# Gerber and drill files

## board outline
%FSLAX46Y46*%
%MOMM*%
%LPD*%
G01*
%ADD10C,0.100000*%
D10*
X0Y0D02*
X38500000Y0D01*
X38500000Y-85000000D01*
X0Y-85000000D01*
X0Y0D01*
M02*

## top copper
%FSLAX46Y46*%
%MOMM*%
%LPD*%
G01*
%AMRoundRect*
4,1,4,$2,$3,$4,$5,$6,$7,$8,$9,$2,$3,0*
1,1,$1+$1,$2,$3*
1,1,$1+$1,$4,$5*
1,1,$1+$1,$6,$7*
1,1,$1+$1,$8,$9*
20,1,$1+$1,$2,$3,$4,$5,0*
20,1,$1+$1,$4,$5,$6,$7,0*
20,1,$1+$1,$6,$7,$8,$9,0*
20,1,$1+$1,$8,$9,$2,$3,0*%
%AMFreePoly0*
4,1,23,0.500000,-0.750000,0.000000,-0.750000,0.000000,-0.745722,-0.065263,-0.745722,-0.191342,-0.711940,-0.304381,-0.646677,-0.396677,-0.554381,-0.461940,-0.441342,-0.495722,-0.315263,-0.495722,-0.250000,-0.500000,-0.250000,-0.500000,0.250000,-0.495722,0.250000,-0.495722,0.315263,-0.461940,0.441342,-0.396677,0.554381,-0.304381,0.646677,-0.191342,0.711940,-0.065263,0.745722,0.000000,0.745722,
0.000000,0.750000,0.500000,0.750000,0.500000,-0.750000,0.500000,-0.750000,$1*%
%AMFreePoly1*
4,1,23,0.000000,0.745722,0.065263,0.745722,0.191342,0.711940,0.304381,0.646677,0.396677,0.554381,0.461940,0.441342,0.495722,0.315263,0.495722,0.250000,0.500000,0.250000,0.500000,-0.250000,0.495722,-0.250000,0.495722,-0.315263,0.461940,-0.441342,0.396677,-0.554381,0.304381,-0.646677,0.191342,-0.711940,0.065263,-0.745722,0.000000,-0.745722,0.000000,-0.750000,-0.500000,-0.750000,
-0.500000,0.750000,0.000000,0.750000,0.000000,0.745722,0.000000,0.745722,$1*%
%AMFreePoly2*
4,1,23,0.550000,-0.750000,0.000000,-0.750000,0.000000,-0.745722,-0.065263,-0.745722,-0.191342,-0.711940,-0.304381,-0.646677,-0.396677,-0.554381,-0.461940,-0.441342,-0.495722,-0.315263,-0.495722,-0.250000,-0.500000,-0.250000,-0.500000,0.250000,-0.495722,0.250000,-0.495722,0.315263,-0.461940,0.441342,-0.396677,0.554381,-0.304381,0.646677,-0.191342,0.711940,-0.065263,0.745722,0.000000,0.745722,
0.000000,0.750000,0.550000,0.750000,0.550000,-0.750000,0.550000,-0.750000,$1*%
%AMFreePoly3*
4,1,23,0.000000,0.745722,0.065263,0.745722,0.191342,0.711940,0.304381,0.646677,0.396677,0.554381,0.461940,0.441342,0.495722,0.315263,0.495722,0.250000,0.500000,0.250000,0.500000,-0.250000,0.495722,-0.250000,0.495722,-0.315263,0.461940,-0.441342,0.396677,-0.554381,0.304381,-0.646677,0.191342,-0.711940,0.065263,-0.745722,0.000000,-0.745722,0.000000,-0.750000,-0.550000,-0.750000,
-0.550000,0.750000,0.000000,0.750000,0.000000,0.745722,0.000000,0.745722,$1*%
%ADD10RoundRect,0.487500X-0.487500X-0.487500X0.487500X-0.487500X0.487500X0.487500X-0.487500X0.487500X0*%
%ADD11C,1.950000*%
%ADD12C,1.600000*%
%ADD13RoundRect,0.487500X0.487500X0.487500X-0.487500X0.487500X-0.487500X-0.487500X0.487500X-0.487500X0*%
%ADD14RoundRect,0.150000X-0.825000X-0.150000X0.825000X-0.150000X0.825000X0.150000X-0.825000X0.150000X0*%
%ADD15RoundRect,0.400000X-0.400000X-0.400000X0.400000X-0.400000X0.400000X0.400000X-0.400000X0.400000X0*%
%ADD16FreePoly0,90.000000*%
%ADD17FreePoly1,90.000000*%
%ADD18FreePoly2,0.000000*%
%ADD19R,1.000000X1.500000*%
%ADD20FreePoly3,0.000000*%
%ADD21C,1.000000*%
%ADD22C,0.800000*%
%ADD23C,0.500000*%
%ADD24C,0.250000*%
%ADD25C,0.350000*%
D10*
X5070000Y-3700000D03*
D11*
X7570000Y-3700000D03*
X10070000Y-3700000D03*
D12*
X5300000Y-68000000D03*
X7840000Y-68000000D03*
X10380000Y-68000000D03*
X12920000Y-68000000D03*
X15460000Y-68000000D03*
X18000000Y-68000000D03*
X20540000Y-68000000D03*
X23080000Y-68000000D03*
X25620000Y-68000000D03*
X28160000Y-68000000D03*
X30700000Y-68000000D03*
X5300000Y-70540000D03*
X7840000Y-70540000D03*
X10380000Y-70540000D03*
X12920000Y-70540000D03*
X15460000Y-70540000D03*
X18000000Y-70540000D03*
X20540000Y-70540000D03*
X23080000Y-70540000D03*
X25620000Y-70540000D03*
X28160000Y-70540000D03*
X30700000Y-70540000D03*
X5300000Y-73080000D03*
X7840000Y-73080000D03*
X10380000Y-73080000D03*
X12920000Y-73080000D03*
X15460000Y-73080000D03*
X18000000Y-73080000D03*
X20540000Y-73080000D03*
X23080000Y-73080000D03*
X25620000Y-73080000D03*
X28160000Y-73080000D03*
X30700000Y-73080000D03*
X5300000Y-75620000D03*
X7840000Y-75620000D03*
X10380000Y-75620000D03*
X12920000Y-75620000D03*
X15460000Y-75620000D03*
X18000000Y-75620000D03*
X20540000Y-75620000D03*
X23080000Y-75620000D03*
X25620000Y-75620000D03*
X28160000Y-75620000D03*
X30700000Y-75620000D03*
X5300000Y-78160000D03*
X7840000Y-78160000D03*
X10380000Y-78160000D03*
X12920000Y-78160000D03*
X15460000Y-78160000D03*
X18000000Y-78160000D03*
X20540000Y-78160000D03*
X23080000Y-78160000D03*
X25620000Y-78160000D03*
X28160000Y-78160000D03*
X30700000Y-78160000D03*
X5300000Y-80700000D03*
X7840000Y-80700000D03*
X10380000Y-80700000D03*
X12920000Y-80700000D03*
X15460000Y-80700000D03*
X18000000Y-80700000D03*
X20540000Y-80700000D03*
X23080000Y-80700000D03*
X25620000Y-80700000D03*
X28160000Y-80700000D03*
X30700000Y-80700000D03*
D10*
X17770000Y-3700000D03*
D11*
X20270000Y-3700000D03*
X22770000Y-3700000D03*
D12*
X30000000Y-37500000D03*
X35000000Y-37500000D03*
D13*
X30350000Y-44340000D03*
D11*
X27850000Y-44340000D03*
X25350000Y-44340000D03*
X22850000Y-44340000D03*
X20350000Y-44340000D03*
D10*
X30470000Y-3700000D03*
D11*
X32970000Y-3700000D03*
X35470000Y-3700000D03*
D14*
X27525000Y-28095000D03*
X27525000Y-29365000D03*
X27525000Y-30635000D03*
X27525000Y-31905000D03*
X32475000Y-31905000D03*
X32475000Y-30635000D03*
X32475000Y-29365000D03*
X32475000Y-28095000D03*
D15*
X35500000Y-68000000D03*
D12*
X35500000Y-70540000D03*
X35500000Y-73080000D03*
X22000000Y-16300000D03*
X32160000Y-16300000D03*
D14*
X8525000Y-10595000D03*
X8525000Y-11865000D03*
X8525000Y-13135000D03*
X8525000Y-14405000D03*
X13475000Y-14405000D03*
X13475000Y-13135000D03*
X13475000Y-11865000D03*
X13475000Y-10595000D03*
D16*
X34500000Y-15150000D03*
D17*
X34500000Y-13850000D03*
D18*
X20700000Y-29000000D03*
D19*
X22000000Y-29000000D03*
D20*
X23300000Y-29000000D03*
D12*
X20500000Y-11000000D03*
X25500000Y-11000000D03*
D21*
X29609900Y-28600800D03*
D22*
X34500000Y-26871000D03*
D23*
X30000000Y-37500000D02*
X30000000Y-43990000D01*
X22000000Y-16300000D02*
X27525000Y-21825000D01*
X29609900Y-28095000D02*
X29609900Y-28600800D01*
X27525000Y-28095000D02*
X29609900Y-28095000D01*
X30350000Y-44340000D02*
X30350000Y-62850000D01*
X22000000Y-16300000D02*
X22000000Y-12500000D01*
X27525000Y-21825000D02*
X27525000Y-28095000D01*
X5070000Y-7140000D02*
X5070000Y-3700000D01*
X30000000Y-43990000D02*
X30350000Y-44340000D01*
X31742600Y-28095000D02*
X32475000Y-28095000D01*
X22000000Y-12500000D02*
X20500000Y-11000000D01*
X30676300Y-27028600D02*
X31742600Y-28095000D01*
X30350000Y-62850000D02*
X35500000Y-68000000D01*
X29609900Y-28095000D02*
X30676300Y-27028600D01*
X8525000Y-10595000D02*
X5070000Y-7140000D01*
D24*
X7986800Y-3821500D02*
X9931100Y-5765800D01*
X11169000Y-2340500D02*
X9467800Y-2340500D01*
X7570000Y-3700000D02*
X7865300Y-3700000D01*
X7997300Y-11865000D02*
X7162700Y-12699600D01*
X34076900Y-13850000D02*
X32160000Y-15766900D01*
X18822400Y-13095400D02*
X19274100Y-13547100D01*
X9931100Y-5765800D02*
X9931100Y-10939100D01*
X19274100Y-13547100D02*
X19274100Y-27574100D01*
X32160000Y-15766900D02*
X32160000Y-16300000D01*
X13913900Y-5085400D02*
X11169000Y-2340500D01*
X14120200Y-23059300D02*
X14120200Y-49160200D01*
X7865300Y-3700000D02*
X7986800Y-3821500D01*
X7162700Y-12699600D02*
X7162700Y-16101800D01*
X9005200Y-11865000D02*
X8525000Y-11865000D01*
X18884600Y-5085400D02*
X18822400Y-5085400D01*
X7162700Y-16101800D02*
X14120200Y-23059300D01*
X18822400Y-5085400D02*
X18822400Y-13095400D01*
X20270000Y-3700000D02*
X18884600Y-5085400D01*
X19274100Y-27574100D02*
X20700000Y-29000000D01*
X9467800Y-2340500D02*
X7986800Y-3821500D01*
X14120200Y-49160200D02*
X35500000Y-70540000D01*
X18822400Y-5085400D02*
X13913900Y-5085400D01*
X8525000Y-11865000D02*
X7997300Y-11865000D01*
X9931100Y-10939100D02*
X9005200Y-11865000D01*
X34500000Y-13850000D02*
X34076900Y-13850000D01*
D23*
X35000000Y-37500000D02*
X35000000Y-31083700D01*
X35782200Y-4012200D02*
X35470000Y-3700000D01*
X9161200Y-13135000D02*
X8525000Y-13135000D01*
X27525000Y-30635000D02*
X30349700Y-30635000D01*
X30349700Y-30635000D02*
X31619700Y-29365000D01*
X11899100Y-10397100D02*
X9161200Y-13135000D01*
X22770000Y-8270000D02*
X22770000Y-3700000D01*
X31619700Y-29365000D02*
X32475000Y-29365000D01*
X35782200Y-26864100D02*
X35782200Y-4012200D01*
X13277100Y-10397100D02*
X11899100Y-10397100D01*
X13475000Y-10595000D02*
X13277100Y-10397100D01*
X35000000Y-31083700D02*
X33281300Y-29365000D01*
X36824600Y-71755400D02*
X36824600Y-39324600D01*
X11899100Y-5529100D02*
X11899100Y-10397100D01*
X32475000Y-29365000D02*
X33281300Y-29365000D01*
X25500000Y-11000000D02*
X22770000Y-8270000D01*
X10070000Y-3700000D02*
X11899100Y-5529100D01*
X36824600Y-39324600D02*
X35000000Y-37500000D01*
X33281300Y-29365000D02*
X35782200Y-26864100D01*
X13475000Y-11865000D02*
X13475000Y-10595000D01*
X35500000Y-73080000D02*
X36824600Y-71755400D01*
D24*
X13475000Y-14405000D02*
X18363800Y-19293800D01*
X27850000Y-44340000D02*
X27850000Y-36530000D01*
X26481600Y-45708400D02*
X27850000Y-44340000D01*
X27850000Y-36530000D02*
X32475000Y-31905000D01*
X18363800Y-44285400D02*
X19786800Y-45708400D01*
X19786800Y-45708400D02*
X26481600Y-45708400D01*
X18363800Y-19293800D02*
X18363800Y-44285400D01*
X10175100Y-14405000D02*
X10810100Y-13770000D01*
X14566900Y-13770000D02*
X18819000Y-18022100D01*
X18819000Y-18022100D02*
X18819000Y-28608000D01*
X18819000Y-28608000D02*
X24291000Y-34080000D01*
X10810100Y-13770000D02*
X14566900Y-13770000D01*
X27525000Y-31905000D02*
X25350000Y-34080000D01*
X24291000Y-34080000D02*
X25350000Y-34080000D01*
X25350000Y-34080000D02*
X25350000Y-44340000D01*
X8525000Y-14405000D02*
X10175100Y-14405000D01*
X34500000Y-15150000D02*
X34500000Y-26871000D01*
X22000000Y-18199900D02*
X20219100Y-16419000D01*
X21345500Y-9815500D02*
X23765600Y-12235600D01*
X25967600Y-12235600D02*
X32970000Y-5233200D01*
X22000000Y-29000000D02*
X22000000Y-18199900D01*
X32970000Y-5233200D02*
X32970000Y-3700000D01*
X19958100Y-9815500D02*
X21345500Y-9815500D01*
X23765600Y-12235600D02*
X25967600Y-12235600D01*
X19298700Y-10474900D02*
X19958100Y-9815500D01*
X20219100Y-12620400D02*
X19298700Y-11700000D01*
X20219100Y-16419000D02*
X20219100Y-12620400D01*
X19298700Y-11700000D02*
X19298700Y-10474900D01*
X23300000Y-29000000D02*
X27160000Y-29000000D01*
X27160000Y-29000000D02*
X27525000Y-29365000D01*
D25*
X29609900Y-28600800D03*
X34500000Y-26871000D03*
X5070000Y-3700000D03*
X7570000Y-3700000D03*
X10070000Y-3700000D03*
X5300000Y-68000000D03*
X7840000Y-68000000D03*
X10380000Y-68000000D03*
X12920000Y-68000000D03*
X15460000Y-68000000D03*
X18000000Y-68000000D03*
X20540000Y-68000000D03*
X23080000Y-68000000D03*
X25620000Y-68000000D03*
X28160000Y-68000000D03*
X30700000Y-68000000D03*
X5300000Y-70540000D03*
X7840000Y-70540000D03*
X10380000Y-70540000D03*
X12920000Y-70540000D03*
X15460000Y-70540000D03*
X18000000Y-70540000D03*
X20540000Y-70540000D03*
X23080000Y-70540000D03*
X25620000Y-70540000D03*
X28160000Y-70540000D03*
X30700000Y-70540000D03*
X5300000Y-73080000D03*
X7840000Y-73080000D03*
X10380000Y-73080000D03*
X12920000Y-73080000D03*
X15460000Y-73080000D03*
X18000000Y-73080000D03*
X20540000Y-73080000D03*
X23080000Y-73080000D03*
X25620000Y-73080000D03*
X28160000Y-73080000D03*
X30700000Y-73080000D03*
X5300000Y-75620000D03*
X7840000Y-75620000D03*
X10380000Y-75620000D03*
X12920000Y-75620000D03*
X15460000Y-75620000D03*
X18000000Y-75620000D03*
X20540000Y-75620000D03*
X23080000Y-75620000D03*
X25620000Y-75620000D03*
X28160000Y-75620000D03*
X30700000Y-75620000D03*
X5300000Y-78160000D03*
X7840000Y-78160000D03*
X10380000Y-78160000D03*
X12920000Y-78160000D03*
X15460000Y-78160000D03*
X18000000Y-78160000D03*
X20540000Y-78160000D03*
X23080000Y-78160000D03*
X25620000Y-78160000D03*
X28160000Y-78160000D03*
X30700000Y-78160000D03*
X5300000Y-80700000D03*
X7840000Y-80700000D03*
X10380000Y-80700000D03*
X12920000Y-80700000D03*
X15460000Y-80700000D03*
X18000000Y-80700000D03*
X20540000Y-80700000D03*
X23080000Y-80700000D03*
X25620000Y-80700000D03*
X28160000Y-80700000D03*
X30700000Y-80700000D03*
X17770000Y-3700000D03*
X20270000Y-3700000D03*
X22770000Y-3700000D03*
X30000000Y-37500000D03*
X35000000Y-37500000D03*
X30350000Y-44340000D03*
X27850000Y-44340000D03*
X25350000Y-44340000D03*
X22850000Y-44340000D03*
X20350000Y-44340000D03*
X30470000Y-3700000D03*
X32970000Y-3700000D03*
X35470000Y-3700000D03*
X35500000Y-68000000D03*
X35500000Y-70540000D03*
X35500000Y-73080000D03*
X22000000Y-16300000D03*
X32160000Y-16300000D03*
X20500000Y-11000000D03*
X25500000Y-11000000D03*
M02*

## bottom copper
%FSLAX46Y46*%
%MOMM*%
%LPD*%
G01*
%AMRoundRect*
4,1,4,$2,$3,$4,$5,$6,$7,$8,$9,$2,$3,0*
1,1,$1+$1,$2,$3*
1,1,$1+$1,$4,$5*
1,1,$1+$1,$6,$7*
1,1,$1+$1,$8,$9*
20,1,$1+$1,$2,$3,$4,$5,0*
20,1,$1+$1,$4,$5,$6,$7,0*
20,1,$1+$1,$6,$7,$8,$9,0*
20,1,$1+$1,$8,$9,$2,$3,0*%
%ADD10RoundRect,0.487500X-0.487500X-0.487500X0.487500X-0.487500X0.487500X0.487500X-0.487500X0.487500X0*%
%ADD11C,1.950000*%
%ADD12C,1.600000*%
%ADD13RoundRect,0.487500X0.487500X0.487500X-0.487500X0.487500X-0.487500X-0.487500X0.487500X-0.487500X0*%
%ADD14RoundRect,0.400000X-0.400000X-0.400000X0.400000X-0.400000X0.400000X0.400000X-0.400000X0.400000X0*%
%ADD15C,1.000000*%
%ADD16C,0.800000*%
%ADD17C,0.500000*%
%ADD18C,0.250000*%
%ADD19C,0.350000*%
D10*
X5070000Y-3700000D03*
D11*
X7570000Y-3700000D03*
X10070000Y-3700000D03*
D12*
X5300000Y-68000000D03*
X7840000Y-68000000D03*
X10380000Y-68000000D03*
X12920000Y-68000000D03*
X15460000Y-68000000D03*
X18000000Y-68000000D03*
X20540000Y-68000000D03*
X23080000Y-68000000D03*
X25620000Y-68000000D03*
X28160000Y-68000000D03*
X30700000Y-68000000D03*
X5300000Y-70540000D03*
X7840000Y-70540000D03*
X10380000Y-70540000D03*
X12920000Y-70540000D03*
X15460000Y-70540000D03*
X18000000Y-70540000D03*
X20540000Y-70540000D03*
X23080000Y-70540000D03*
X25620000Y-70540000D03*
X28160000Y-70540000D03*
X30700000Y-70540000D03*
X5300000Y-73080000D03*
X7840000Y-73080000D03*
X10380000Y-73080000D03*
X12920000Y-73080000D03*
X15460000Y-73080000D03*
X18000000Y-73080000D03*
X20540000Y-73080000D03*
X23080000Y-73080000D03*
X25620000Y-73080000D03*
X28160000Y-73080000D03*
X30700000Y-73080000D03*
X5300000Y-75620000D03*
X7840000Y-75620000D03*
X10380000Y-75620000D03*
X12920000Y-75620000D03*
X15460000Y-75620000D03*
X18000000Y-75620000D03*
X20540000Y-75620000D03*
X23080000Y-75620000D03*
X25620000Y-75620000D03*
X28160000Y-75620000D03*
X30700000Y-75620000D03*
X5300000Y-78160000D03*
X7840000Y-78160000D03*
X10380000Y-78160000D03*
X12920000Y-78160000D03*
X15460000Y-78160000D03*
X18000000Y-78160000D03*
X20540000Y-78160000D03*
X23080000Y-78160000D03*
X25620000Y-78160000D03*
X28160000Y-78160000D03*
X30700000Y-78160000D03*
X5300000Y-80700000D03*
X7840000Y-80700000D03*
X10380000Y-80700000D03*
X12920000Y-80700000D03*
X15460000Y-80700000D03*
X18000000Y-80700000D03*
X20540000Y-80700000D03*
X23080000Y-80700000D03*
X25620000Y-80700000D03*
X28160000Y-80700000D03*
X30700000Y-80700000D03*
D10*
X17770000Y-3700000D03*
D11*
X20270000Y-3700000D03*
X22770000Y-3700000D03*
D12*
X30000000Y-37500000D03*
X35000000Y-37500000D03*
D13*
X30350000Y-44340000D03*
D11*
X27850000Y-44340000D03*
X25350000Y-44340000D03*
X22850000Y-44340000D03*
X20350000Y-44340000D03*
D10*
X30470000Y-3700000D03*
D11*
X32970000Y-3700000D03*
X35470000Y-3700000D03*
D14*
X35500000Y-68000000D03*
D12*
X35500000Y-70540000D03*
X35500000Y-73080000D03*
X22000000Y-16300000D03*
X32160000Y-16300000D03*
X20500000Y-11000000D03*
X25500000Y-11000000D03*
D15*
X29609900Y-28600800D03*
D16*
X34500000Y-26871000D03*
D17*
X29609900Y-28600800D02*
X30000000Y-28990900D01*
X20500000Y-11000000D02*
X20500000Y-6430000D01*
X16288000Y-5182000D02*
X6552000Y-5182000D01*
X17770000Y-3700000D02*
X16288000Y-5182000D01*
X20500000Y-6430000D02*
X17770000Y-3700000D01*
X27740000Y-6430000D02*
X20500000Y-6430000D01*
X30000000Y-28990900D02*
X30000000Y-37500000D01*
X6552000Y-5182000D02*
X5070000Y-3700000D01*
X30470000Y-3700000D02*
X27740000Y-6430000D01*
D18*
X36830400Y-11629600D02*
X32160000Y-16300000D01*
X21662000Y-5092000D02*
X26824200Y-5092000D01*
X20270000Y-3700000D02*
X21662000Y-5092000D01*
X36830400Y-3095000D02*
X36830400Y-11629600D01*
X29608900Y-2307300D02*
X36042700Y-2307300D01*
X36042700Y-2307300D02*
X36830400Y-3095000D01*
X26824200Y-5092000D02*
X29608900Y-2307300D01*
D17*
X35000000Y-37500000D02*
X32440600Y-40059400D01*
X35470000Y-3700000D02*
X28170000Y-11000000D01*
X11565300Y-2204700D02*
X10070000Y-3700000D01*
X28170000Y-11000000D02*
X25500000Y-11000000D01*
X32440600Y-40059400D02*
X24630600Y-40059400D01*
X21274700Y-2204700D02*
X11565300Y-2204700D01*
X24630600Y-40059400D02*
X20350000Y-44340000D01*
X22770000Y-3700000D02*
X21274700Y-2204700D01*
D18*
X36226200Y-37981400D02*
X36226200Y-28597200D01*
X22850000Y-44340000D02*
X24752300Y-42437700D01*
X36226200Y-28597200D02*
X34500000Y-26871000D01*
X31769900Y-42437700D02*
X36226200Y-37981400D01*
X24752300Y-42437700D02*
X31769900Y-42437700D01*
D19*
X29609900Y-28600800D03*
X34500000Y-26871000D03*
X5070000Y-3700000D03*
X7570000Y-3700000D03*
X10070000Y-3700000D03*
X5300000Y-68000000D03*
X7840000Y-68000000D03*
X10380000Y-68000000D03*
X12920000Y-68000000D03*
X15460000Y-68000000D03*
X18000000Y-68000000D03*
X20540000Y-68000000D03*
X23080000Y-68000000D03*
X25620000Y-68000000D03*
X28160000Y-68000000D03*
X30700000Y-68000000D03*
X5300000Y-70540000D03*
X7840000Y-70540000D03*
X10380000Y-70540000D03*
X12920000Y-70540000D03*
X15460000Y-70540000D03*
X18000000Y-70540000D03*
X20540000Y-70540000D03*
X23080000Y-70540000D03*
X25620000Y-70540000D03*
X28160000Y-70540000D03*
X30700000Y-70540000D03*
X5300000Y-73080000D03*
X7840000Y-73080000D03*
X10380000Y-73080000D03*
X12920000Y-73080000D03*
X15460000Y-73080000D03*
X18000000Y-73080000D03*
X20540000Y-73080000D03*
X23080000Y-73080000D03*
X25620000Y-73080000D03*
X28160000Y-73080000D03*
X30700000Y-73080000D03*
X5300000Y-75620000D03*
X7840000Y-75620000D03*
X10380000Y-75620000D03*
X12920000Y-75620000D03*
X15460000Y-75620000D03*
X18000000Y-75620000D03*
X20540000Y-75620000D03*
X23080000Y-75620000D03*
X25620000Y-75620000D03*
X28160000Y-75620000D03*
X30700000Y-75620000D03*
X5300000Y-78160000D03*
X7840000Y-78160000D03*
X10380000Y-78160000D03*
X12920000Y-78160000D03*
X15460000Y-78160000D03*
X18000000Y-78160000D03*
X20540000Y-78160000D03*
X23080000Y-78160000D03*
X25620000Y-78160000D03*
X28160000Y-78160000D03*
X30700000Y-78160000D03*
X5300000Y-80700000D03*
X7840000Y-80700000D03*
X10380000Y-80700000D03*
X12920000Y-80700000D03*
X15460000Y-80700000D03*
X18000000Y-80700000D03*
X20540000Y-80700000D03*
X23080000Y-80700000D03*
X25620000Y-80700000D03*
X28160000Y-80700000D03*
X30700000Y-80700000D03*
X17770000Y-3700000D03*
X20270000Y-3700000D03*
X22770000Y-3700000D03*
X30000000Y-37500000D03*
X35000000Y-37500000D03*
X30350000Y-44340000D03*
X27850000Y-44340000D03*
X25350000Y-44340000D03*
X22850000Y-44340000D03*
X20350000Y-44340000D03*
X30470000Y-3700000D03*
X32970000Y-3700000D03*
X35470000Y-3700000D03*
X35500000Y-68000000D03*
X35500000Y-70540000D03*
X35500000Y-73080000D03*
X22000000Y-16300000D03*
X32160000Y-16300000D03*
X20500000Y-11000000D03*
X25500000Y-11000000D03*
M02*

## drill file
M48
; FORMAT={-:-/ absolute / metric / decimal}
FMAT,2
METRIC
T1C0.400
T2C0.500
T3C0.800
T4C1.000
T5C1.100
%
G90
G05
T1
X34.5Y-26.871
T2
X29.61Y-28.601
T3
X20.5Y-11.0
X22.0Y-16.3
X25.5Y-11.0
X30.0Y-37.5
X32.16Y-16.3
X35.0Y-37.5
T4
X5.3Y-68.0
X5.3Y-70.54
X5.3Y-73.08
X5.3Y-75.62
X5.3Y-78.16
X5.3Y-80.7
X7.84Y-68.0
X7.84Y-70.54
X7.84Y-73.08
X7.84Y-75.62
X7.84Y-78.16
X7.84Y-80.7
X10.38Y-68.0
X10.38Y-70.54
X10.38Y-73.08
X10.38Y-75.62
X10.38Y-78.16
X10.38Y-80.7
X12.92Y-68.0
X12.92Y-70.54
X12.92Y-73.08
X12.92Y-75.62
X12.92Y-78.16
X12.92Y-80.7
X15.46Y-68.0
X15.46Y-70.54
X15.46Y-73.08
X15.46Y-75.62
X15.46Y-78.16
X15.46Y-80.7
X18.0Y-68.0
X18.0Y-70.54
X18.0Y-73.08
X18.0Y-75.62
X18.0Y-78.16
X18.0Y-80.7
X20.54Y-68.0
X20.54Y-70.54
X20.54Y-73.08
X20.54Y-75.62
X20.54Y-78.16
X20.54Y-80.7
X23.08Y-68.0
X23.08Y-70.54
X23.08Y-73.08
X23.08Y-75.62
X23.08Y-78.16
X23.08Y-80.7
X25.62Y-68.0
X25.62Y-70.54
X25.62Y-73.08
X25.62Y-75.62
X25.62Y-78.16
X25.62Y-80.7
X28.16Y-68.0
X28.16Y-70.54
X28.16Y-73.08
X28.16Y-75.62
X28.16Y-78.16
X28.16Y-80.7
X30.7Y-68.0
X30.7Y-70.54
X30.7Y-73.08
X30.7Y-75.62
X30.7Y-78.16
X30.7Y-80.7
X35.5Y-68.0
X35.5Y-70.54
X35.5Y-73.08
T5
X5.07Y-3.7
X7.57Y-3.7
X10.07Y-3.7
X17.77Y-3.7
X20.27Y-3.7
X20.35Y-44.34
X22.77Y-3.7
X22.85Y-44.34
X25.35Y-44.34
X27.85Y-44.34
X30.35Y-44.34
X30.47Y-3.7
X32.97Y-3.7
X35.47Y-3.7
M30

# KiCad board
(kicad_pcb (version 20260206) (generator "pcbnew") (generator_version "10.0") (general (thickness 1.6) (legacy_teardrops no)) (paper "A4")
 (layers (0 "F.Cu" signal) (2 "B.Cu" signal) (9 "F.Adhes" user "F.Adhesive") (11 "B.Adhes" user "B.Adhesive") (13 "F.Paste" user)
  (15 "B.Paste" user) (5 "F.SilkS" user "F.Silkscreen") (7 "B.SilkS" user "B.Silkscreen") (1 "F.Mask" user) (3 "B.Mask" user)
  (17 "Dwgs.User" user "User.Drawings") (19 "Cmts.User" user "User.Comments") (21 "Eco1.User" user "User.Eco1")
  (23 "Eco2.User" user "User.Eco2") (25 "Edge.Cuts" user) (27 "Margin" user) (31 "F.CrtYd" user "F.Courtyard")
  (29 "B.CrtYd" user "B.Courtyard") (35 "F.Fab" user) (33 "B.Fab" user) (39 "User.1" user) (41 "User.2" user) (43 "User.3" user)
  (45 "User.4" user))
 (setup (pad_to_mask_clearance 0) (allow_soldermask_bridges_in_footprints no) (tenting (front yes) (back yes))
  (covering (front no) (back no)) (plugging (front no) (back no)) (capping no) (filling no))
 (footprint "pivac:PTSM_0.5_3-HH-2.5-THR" (layer "F.Cu") (at 7.57 3.7)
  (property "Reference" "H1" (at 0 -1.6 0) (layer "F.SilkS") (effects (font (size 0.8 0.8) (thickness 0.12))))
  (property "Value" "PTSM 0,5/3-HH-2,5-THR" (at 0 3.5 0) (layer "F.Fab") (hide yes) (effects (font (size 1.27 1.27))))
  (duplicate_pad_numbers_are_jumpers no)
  (pad "1" thru_hole roundrect (at -2.5 0) (size 1.95 1.95) (drill 1.1) (layers "*.Cu" "*.Mask") (remove_unused_layers no)
   (roundrect_rratio 0.25) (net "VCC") (thermal_bridge_angle 45))
  (pad "2" thru_hole circle (at 0 0) (size 1.95 1.95) (drill 1.1) (layers "*.Cu" "*.Mask") (remove_unused_layers no) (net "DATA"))
  (pad "3" thru_hole circle (at 2.5 0) (size 1.95 1.95) (drill 1.1) (layers "*.Cu" "*.Mask") (remove_unused_layers no) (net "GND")))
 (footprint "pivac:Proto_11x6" (layer "F.Cu") (at 5.3 68)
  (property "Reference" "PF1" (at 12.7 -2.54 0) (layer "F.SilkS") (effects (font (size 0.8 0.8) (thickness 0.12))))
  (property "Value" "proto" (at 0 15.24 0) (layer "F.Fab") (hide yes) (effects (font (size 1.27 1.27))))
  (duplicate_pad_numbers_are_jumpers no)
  (pad "1" thru_hole circle (at 0 0) (size 1.6 1.6) (drill 1) (layers "*.Cu" "*.Mask") (remove_unused_layers no))
  (pad "2" thru_hole circle (at 2.54 0) (size 1.6 1.6) (drill 1) (layers "*.Cu" "*.Mask") (remove_unused_layers no))
  (pad "3" thru_hole circle (at 5.08 0) (size 1.6 1.6) (drill 1) (layers "*.Cu" "*.Mask") (remove_unused_layers no))
  (pad "4" thru_hole circle (at 7.62 0) (size 1.6 1.6) (drill 1) (layers "*.Cu" "*.Mask") (remove_unused_layers no))
  (pad "5" thru_hole circle (at 10.16 0) (size 1.6 1.6) (drill 1) (layers "*.Cu" "*.Mask") (remove_unused_layers no))
  (pad "6" thru_hole circle (at 12.7 0) (size 1.6 1.6) (drill 1) (layers "*.Cu" "*.Mask") (remove_unused_layers no))
  (pad "7" thru_hole circle (at 15.24 0) (size 1.6 1.6) (drill 1) (layers "*.Cu" "*.Mask") (remove_unused_layers no))
  (pad "8" thru_hole circle (at 17.78 0) (size 1.6 1.6) (drill 1) (layers "*.Cu" "*.Mask") (remove_unused_layers no))
  (pad "9" thru_hole circle (at 20.32 0) (size 1.6 1.6) (drill 1) (layers "*.Cu" "*.Mask") (remove_unused_layers no))
  (pad "10" thru_hole circle (at 22.86 0) (size 1.6 1.6) (drill 1) (layers "*.Cu" "*.Mask") (remove_unused_layers no))
  (pad "11" thru_hole circle (at 25.4 0) (size 1.6 1.6) (drill 1) (layers "*.Cu" "*.Mask") (remove_unused_layers no))
  (pad "12" thru_hole circle (at 0 2.54) (size 1.6 1.6) (drill 1) (layers "*.Cu" "*.Mask") (remove_unused_layers no))
  (pad "13" thru_hole circle (at 2.54 2.54) (size 1.6 1.6) (drill 1) (layers "*.Cu" "*.Mask") (remove_unused_layers no))
  (pad "14" thru_hole circle (at 5.08 2.54) (size 1.6 1.6) (drill 1) (layers "*.Cu" "*.Mask") (remove_unused_layers no))
  (pad "15" thru_hole circle (at 7.62 2.54) (size 1.6 1.6) (drill 1) (layers "*.Cu" "*.Mask") (remove_unused_layers no))
  (pad "16" thru_hole circle (at 10.16 2.54) (size 1.6 1.6) (drill 1) (layers "*.Cu" "*.Mask") (remove_unused_layers no))
  (pad "17" thru_hole circle (at 12.7 2.54) (size 1.6 1.6) (drill 1) (layers "*.Cu" "*.Mask") (remove_unused_layers no))
  (pad "18" thru_hole circle (at 15.24 2.54) (size 1.6 1.6) (drill 1) (layers "*.Cu" "*.Mask") (remove_unused_layers no))
  (pad "19" thru_hole circle (at 17.78 2.54) (size 1.6 1.6) (drill 1) (layers "*.Cu" "*.Mask") (remove_unused_layers no))
  (pad "20" thru_hole circle (at 20.32 2.54) (size 1.6 1.6) (drill 1) (layers "*.Cu" "*.Mask") (remove_unused_layers no))
  (pad "21" thru_hole circle (at 22.86 2.54) (size 1.6 1.6) (drill 1) (layers "*.Cu" "*.Mask") (remove_unused_layers no))
  (pad "22" thru_hole circle (at 25.4 2.54) (size 1.6 1.6) (drill 1) (layers "*.Cu" "*.Mask") (remove_unused_layers no))
  (pad "23" thru_hole circle (at 0 5.08) (size 1.6 1.6) (drill 1) (layers "*.Cu" "*.Mask") (remove_unused_layers no))
  (pad "24" thru_hole circle (at 2.54 5.08) (size 1.6 1.6) (drill 1) (layers "*.Cu" "*.Mask") (remove_unused_layers no))
  (pad "25" thru_hole circle (at 5.08 5.08) (size 1.6 1.6) (drill 1) (layers "*.Cu" "*.Mask") (remove_unused_layers no))
  (pad "26" thru_hole circle (at 7.62 5.08) (size 1.6 1.6) (drill 1) (layers "*.Cu" "*.Mask") (remove_unused_layers no))
  (pad "27" thru_hole circle (at 10.16 5.08) (size 1.6 1.6) (drill 1) (layers "*.Cu" "*.Mask") (remove_unused_layers no))
  (pad "28" thru_hole circle (at 12.7 5.08) (size 1.6 1.6) (drill 1) (layers "*.Cu" "*.Mask") (remove_unused_layers no))
  (pad "29" thru_hole circle (at 15.24 5.08) (size 1.6 1.6) (drill 1) (layers "*.Cu" "*.Mask") (remove_unused_layers no))
  (pad "30" thru_hole circle (at 17.78 5.08) (size 1.6 1.6) (drill 1) (layers "*.Cu" "*.Mask") (remove_unused_layers no))
  (pad "31" thru_hole circle (at 20.32 5.08) (size 1.6 1.6) (drill 1) (layers "*.Cu" "*.Mask") (remove_unused_layers no))
  (pad "32" thru_hole circle (at 22.86 5.08) (size 1.6 1.6) (drill 1) (layers "*.Cu" "*.Mask") (remove_unused_layers no))
  (pad "33" thru_hole circle (at 25.4 5.08) (size 1.6 1.6) (drill 1) (layers "*.Cu" "*.Mask") (remove_unused_layers no))
  (pad "34" thru_hole circle (at 0 7.62) (size 1.6 1.6) (drill 1) (layers "*.Cu" "*.Mask") (remove_unused_layers no))
  (pad "35" thru_hole circle (at 2.54 7.62) (size 1.6 1.6) (drill 1) (layers "*.Cu" "*.Mask") (remove_unused_layers no))
  (pad "36" thru_hole circle (at 5.08 7.62) (size 1.6 1.6) (drill 1) (layers "*.Cu" "*.Mask") (remove_unused_layers no))
  (pad "37" thru_hole circle (at 7.62 7.62) (size 1.6 1.6) (drill 1) (layers "*.Cu" "*.Mask") (remove_unused_layers no))
  (pad "38" thru_hole circle (at 10.16 7.62) (size 1.6 1.6) (drill 1) (layers "*.Cu" "*.Mask") (remove_unused_layers no))
  (pad "39" thru_hole circle (at 12.7 7.62) (size 1.6 1.6) (drill 1) (layers "*.Cu" "*.Mask") (remove_unused_layers no))
  (pad "40" thru_hole circle (at 15.24 7.62) (size 1.6 1.6) (drill 1) (layers "*.Cu" "*.Mask") (remove_unused_layers no))
  (pad "41" thru_hole circle (at 17.78 7.62) (size 1.6 1.6) (drill 1) (layers "*.Cu" "*.Mask") (remove_unused_layers no))
  (pad "42" thru_hole circle (at 20.32 7.62) (size 1.6 1.6) (drill 1) (layers "*.Cu" "*.Mask") (remove_unused_layers no))
  (pad "43" thru_hole circle (at 22.86 7.62) (size 1.6 1.6) (drill 1) (layers "*.Cu" "*.Mask") (remove_unused_layers no))
  (pad "44" thru_hole circle (at 25.4 7.62) (size 1.6 1.6) (drill 1) (layers "*.Cu" "*.Mask") (remove_unused_layers no))
  (pad "45" thru_hole circle (at 0 10.16) (size 1.6 1.6) (drill 1) (layers "*.Cu" "*.Mask") (remove_unused_layers no))
  (pad "46" thru_hole circle (at 2.54 10.16) (size 1.6 1.6) (drill 1) (layers "*.Cu" "*.Mask") (remove_unused_layers no))
  (pad "47" thru_hole circle (at 5.08 10.16) (size 1.6 1.6) (drill 1) (layers "*.Cu" "*.Mask") (remove_unused_layers no))
  (pad "48" thru_hole circle (at 7.62 10.16) (size 1.6 1.6) (drill 1) (layers "*.Cu" "*.Mask") (remove_unused_layers no))
  (pad "49" thru_hole circle (at 10.16 10.16) (size 1.6 1.6) (drill 1) (layers "*.Cu" "*.Mask") (remove_unused_layers no))
  (pad "50" thru_hole circle (at 12.7 10.16) (size 1.6 1.6) (drill 1) (layers "*.Cu" "*.Mask") (remove_unused_layers no))
  (pad "51" thru_hole circle (at 15.24 10.16) (size 1.6 1.6) (drill 1) (layers "*.Cu" "*.Mask") (remove_unused_layers no))
  (pad "52" thru_hole circle (at 17.78 10.16) (size 1.6 1.6) (drill 1) (layers "*.Cu" "*.Mask") (remove_unused_layers no))
  (pad "53" thru_hole circle (at 20.32 10.16) (size 1.6 1.6) (drill 1) (layers "*.Cu" "*.Mask") (remove_unused_layers no))
  (pad "54" thru_hole circle (at 22.86 10.16) (size 1.6 1.6) (drill 1) (layers "*.Cu" "*.Mask") (remove_unused_layers no))
  (pad "55" thru_hole circle (at 25.4 10.16) (size 1.6 1.6) (drill 1) (layers "*.Cu" "*.Mask") (remove_unused_layers no))
  (pad "56" thru_hole circle (at 0 12.7) (size 1.6 1.6) (drill 1) (layers "*.Cu" "*.Mask") (remove_unused_layers no))
  (pad "57" thru_hole circle (at 2.54 12.7) (size 1.6 1.6) (drill 1) (layers "*.Cu" "*.Mask") (remove_unused_layers no))
  (pad "58" thru_hole circle (at 5.08 12.7) (size 1.6 1.6) (drill 1) (layers "*.Cu" "*.Mask") (remove_unused_layers no))
  (pad "59" thru_hole circle (at 7.62 12.7) (size 1.6 1.6) (drill 1) (layers "*.Cu" "*.Mask") (remove_unused_layers no))
  (pad "60" thru_hole circle (at 10.16 12.7) (size 1.6 1.6) (drill 1) (layers "*.Cu" "*.Mask") (remove_unused_layers no))
  (pad "61" thru_hole circle (at 12.7 12.7) (size 1.6 1.6) (drill 1) (layers "*.Cu" "*.Mask") (remove_unused_layers no))
  (pad "62" thru_hole circle (at 15.24 12.7) (size 1.6 1.6) (drill 1) (layers "*.Cu" "*.Mask") (remove_unused_layers no))
  (pad "63" thru_hole circle (at 17.78 12.7) (size 1.6 1.6) (drill 1) (layers "*.Cu" "*.Mask") (remove_unused_layers no))
  (pad "64" thru_hole circle (at 20.32 12.7) (size 1.6 1.6) (drill 1) (layers "*.Cu" "*.Mask") (remove_unused_layers no))
  (pad "65" thru_hole circle (at 22.86 12.7) (size 1.6 1.6) (drill 1) (layers "*.Cu" "*.Mask") (remove_unused_layers no))
  (pad "66" thru_hole circle (at 25.4 12.7) (size 1.6 1.6) (drill 1) (layers "*.Cu" "*.Mask") (remove_unused_layers no)))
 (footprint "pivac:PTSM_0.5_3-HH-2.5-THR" (layer "F.Cu") (at 20.27 3.7)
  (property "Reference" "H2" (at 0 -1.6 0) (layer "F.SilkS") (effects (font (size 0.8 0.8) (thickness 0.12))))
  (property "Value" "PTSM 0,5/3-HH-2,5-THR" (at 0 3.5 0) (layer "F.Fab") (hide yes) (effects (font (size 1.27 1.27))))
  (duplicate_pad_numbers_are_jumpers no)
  (pad "1" thru_hole roundrect (at -2.5 0) (size 1.95 1.95) (drill 1.1) (layers "*.Cu" "*.Mask") (remove_unused_layers no)
   (roundrect_rratio 0.25) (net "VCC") (thermal_bridge_angle 45))
  (pad "2" thru_hole circle (at 0 0) (size 1.95 1.95) (drill 1.1) (layers "*.Cu" "*.Mask") (remove_unused_layers no) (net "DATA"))
  (pad "3" thru_hole circle (at 2.5 0) (size 1.95 1.95) (drill 1.1) (layers "*.Cu" "*.Mask") (remove_unused_layers no) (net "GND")))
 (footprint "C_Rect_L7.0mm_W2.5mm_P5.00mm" (layer "F.Cu") (at 30 37.5)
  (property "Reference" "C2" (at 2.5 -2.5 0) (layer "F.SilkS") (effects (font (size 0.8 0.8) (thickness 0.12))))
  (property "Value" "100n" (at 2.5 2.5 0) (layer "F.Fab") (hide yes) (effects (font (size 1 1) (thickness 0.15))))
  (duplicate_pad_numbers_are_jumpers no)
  (pad "1" thru_hole circle (at 0 0) (size 1.6 1.6) (drill 0.8) (layers "*.Cu" "*.Mask") (remove_unused_layers no) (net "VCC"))
  (pad "2" thru_hole circle (at 5 0) (size 1.6 1.6) (drill 0.8) (layers "*.Cu" "*.Mask") (remove_unused_layers no) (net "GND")))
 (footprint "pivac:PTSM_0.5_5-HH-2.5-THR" (layer "F.Cu") (at 25.35 44.34 180)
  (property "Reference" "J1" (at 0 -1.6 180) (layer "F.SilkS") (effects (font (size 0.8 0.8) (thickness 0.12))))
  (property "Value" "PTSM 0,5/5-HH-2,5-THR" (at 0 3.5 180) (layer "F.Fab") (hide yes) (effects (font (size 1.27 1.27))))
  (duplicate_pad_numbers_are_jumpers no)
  (pad "1" thru_hole roundrect (at -5 0 180) (size 1.95 1.95) (drill 1.1) (layers "*.Cu" "*.Mask") (remove_unused_layers no)
   (roundrect_rratio 0.25) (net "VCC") (thermal_bridge_angle 45))
  (pad "2" thru_hole circle (at -2.5 0 180) (size 1.95 1.95) (drill 1.1) (layers "*.Cu" "*.Mask") (remove_unused_layers no) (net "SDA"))
  (pad "3" thru_hole circle (at 0 0 180) (size 1.95 1.95) (drill 1.1) (layers "*.Cu" "*.Mask") (remove_unused_layers no) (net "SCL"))
  (pad "4" thru_hole circle (at 2.5 0 180) (size 1.95 1.95) (drill 1.1) (layers "*.Cu" "*.Mask") (remove_unused_layers no) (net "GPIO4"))
  (pad "5" thru_hole circle (at 5 0 180) (size 1.95 1.95) (drill 1.1) (layers "*.Cu" "*.Mask") (remove_unused_layers no) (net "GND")))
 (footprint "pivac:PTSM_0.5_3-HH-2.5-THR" (layer "F.Cu") (at 32.97 3.7)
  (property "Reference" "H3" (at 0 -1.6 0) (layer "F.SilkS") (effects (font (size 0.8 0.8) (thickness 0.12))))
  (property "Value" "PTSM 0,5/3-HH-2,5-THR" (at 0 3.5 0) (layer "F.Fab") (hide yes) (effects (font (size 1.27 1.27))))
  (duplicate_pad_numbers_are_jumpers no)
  (pad "1" thru_hole roundrect (at -2.5 0) (size 1.95 1.95) (drill 1.1) (layers "*.Cu" "*.Mask") (remove_unused_layers no)
   (roundrect_rratio 0.25) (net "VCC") (thermal_bridge_angle 45))
  (pad "2" thru_hole circle (at 0 0) (size 1.95 1.95) (drill 1.1) (layers "*.Cu" "*.Mask") (remove_unused_layers no) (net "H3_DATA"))
  (pad "3" thru_hole circle (at 2.5 0) (size 1.95 1.95) (drill 1.1) (layers "*.Cu" "*.Mask") (remove_unused_layers no) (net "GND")))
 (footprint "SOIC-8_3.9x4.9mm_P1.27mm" (layer "F.Cu") (at 30 30)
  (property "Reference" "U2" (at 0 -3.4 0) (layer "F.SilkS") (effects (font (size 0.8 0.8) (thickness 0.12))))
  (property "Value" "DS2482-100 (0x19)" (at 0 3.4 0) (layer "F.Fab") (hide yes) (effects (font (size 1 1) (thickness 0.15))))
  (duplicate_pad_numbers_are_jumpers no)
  (pad "1" smd roundrect (at -2.475 -1.905) (size 1.95 0.6) (layers "F.Cu" "F.Mask" "F.Paste") (roundrect_rratio 0.25) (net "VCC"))
  (pad "2" smd roundrect (at -2.475 -0.635) (size 1.95 0.6) (layers "F.Cu" "F.Mask" "F.Paste") (roundrect_rratio 0.25) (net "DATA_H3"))
  (pad "3" smd roundrect (at -2.475 0.635) (size 1.95 0.6) (layers "F.Cu" "F.Mask" "F.Paste") (roundrect_rratio 0.25) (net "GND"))
  (pad "4" smd roundrect (at -2.475 1.905) (size 1.95 0.6) (layers "F.Cu" "F.Mask" "F.Paste") (roundrect_rratio 0.25) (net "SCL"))
  (pad "5" smd roundrect (at 2.475 1.905) (size 1.95 0.6) (layers "F.Cu" "F.Mask" "F.Paste") (roundrect_rratio 0.25) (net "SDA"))
  (pad "6" smd roundrect (at 2.475 0.635) (size 1.95 0.6) (layers "F.Cu" "F.Mask" "F.Paste") (roundrect_rratio 0.25))
  (pad "7" smd roundrect (at 2.475 -0.635) (size 1.95 0.6) (layers "F.Cu" "F.Mask" "F.Paste") (roundrect_rratio 0.25) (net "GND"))
  (pad "8" smd roundrect (at 2.475 -1.905) (size 1.95 0.6) (layers "F.Cu" "F.Mask" "F.Paste") (roundrect_rratio 0.25) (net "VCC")))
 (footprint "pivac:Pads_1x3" (layer "F.Cu") (at 35.5 68)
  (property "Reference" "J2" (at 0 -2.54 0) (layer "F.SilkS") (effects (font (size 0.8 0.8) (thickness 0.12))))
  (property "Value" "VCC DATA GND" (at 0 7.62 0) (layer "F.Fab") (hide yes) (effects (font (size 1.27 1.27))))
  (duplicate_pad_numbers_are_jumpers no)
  (pad "1" thru_hole roundrect (at 0 0) (size 1.6 1.6) (drill 1) (layers "*.Cu" "*.Mask") (remove_unused_layers no) (roundrect_rratio 0.25)
   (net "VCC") (thermal_bridge_angle 45))
  (pad "2" thru_hole circle (at 0 2.54) (size 1.6 1.6) (drill 1) (layers "*.Cu" "*.Mask") (remove_unused_layers no) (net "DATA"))
  (pad "3" thru_hole circle (at 0 5.08) (size 1.6 1.6) (drill 1) (layers "*.Cu" "*.Mask") (remove_unused_layers no) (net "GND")))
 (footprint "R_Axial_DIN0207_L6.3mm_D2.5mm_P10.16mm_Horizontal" (layer "F.Cu") (at 22 16.3)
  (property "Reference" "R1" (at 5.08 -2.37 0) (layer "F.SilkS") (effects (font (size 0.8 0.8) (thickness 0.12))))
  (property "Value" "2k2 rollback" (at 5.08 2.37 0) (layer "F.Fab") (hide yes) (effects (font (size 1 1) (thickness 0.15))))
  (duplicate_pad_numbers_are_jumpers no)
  (pad "1" thru_hole circle (at 0 0) (size 1.6 1.6) (drill 0.8) (layers "*.Cu" "*.Mask") (remove_unused_layers no) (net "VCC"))
  (pad "2" thru_hole circle (at 10.16 0) (size 1.6 1.6) (drill 0.8) (layers "*.Cu" "*.Mask") (remove_unused_layers no) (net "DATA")))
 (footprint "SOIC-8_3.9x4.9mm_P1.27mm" (layer "F.Cu") (at 11 12.5)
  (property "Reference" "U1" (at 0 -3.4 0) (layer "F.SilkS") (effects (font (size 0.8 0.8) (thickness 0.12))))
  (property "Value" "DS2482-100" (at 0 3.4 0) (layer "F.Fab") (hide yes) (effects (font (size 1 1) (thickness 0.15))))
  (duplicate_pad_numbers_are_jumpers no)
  (pad "1" smd roundrect (at -2.475 -1.905) (size 1.95 0.6) (layers "F.Cu" "F.Mask" "F.Paste") (roundrect_rratio 0.25) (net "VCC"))
  (pad "2" smd roundrect (at -2.475 -0.635) (size 1.95 0.6) (layers "F.Cu" "F.Mask" "F.Paste") (roundrect_rratio 0.25) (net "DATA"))
  (pad "3" smd roundrect (at -2.475 0.635) (size 1.95 0.6) (layers "F.Cu" "F.Mask" "F.Paste") (roundrect_rratio 0.25) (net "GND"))
  (pad "4" smd roundrect (at -2.475 1.905) (size 1.95 0.6) (layers "F.Cu" "F.Mask" "F.Paste") (roundrect_rratio 0.25) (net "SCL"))
  (pad "5" smd roundrect (at 2.475 1.905) (size 1.95 0.6) (layers "F.Cu" "F.Mask" "F.Paste") (roundrect_rratio 0.25) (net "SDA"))
  (pad "6" smd roundrect (at 2.475 0.635) (size 1.95 0.6) (layers "F.Cu" "F.Mask" "F.Paste") (roundrect_rratio 0.25))
  (pad "7" smd roundrect (at 2.475 -0.635) (size 1.95 0.6) (layers "F.Cu" "F.Mask" "F.Paste") (roundrect_rratio 0.25) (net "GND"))
  (pad "8" smd roundrect (at 2.475 -1.905) (size 1.95 0.6) (layers "F.Cu" "F.Mask" "F.Paste") (roundrect_rratio 0.25) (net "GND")))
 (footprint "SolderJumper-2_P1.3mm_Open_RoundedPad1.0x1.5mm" (layer "F.Cu") (at 34.5 14.5 90)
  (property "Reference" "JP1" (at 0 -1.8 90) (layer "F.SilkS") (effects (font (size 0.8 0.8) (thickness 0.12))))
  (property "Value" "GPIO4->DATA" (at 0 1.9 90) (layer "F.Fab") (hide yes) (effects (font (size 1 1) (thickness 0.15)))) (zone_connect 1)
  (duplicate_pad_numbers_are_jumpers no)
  (pad "1" smd custom (at -0.65 0 90) (size 1 0.5) (layers "F.Cu" "F.Mask") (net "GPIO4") (zone_connect 2) (thermal_bridge_angle 45)
   (options (clearance outline) (anchor rect)) (primitives))
  (pad "2" smd custom (at 0.65 0 90) (size 1 0.5) (layers "F.Cu" "F.Mask") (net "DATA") (zone_connect 2) (thermal_bridge_angle 45)
   (options (clearance outline) (anchor rect)) (primitives)))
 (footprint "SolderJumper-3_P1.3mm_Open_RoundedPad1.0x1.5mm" (layer "F.Cu") (at 22 29)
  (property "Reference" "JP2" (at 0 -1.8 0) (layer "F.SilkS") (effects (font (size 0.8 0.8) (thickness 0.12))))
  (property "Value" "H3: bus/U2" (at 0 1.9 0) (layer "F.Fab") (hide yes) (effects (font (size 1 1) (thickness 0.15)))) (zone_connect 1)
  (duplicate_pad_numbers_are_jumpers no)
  (pad "1" smd custom (at -1.3 0) (size 1 0.5) (layers "F.Cu" "F.Mask") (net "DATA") (zone_connect 2) (thermal_bridge_angle 45)
   (options (clearance outline) (anchor rect)) (primitives))
  (pad "2" smd rect (at 0 0) (size 1 1.5) (layers "F.Cu" "F.Mask") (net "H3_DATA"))
  (pad "3" smd custom (at 1.3 0) (size 1 0.5) (layers "F.Cu" "F.Mask") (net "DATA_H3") (zone_connect 2) (thermal_bridge_angle 45)
   (options (clearance outline) (anchor rect)) (primitives)))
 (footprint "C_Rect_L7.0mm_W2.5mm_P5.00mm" (layer "F.Cu") (at 20.5 11)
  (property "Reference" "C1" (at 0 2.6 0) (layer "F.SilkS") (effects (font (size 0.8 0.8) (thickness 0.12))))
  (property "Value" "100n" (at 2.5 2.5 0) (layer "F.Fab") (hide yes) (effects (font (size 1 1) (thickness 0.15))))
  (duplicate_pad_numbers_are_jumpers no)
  (pad "1" thru_hole circle (at 0 0) (size 1.6 1.6) (drill 0.8) (layers "*.Cu" "*.Mask") (remove_unused_layers no) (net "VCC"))
  (pad "2" thru_hole circle (at 5 0) (size 1.6 1.6) (drill 0.8) (layers "*.Cu" "*.Mask") (remove_unused_layers no) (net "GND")))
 (gr_rect (start 0 0) (end 38.5 85) (stroke (width 0.1) (type default)) (fill no) (layer "Edge.Cuts"))
 (segment (start 30 37.5) (end 30 43.99) (width 0.5) (layer "F.Cu") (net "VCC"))
 (segment (start 22 16.3) (end 27.525 21.825) (width 0.5) (layer "F.Cu") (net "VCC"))
 (segment (start 29.6099 28.095) (end 29.6099 28.6008) (width 0.5) (layer "F.Cu") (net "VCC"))
 (segment (start 27.525 28.095) (end 29.6099 28.095) (width 0.5) (layer "F.Cu") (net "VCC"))
 (segment (start 30.35 44.34) (end 30.35 62.85) (width 0.5) (layer "F.Cu") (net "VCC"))
 (segment (start 22 16.3) (end 22 12.5) (width 0.5) (layer "F.Cu") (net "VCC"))
 (segment (start 27.525 21.825) (end 27.525 28.095) (width 0.5) (layer "F.Cu") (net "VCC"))
 (segment (start 5.07 7.14) (end 5.07 3.7) (width 0.5) (layer "F.Cu") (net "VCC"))
 (segment (start 30 43.99) (end 30.35 44.34) (width 0.5) (layer "F.Cu") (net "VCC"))
 (segment (start 31.7426 28.095) (end 32.475 28.095) (width 0.5) (layer "F.Cu") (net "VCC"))
 (segment (start 22 12.5) (end 20.5 11) (width 0.5) (layer "F.Cu") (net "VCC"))
 (segment (start 30.6763 27.0286) (end 31.7426 28.095) (width 0.5) (layer "F.Cu") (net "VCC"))
 (segment (start 30.35 62.85) (end 35.5 68) (width 0.5) (layer "F.Cu") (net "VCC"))
 (segment (start 29.6099 28.095) (end 30.6763 27.0286) (width 0.5) (layer "F.Cu") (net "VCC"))
 (segment (start 8.525 10.595) (end 5.07 7.14) (width 0.5) (layer "F.Cu") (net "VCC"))
 (via (at 29.6099 28.6008) (size 1) (drill 0.5) (layers "F.Cu" "B.Cu") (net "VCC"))
 (segment (start 29.6099 28.6008) (end 30 28.9909) (width 0.5) (layer "B.Cu") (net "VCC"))
 (segment (start 20.5 11) (end 20.5 6.43) (width 0.5) (layer "B.Cu") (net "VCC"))
 (segment (start 16.288 5.182) (end 6.552 5.182) (width 0.5) (layer "B.Cu") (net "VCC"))
 (segment (start 17.77 3.7) (end 16.288 5.182) (width 0.5) (layer "B.Cu") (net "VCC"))
 (segment (start 20.5 6.43) (end 17.77 3.7) (width 0.5) (layer "B.Cu") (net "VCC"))
 (segment (start 27.74 6.43) (end 20.5 6.43) (width 0.5) (layer "B.Cu") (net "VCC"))
 (segment (start 30 28.9909) (end 30 37.5) (width 0.5) (layer "B.Cu") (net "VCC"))
 (segment (start 6.552 5.182) (end 5.07 3.7) (width 0.5) (layer "B.Cu") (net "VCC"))
 (segment (start 30.47 3.7) (end 27.74 6.43) (width 0.5) (layer "B.Cu") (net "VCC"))
 (segment (start 7.9868 3.8215) (end 9.9311 5.7658) (width 0.25) (layer "F.Cu") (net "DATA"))
 (segment (start 11.169 2.3405) (end 9.4678 2.3405) (width 0.25) (layer "F.Cu") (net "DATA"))
 (segment (start 7.57 3.7) (end 7.8653 3.7) (width 0.25) (layer "F.Cu") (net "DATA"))
 (segment (start 7.9973 11.865) (end 7.1627 12.6996) (width 0.25) (layer "F.Cu") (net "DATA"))
 (segment (start 34.0769 13.85) (end 32.16 15.7669) (width 0.25) (layer "F.Cu") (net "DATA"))
 (segment (start 18.8224 13.0954) (end 19.2741 13.5471) (width 0.25) (layer "F.Cu") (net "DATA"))
 (segment (start 9.9311 5.7658) (end 9.9311 10.9391) (width 0.25) (layer "F.Cu") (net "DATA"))
 (segment (start 19.2741 13.5471) (end 19.2741 27.5741) (width 0.25) (layer "F.Cu") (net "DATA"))
 (segment (start 32.16 15.7669) (end 32.16 16.3) (width 0.25) (layer "F.Cu") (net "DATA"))
 (segment (start 13.9139 5.0854) (end 11.169 2.3405) (width 0.25) (layer "F.Cu") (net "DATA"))
 (segment (start 14.1202 23.0593) (end 14.1202 49.1602) (width 0.25) (layer "F.Cu") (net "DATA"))
 (segment (start 7.8653 3.7) (end 7.9868 3.8215) (width 0.25) (layer "F.Cu") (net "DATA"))
 (segment (start 7.1627 12.6996) (end 7.1627 16.1018) (width 0.25) (layer "F.Cu") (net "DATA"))
 (segment (start 9.0052 11.865) (end 8.525 11.865) (width 0.25) (layer "F.Cu") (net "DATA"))
 (segment (start 18.8846 5.0854) (end 18.8224 5.0854) (width 0.25) (layer "F.Cu") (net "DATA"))
 (segment (start 7.1627 16.1018) (end 14.1202 23.0593) (width 0.25) (layer "F.Cu") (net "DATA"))
 (segment (start 18.8224 5.0854) (end 18.8224 13.0954) (width 0.25) (layer "F.Cu") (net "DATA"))
 (segment (start 20.27 3.7) (end 18.8846 5.0854) (width 0.25) (layer "F.Cu") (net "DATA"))
 (segment (start 19.2741 27.5741) (end 20.7 29) (width 0.25) (layer "F.Cu") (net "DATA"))
 (segment (start 9.4678 2.3405) (end 7.9868 3.8215) (width 0.25) (layer "F.Cu") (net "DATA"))
 (segment (start 14.1202 49.1602) (end 35.5 70.54) (width 0.25) (layer "F.Cu") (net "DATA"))
 (segment (start 18.8224 5.0854) (end 13.9139 5.0854) (width 0.25) (layer "F.Cu") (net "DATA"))
 (segment (start 8.525 11.865) (end 7.9973 11.865) (width 0.25) (layer "F.Cu") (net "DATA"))
 (segment (start 9.9311 10.9391) (end 9.0052 11.865) (width 0.25) (layer "F.Cu") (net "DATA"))
 (segment (start 34.5 13.85) (end 34.0769 13.85) (width 0.25) (layer "F.Cu") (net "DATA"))
 (segment (start 36.8304 11.6296) (end 32.16 16.3) (width 0.25) (layer "B.Cu") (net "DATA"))
 (segment (start 21.662 5.092) (end 26.8242 5.092) (width 0.25) (layer "B.Cu") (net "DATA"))
 (segment (start 20.27 3.7) (end 21.662 5.092) (width 0.25) (layer "B.Cu") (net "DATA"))
 (segment (start 36.8304 3.095) (end 36.8304 11.6296) (width 0.25) (layer "B.Cu") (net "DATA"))
 (segment (start 29.6089 2.3073) (end 36.0427 2.3073) (width 0.25) (layer "B.Cu") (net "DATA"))
 (segment (start 36.0427 2.3073) (end 36.8304 3.095) (width 0.25) (layer "B.Cu") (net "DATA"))
 (segment (start 26.8242 5.092) (end 29.6089 2.3073) (width 0.25) (layer "B.Cu") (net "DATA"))
 (segment (start 35 37.5) (end 35 31.0837) (width 0.5) (layer "F.Cu") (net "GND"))
 (segment (start 35.7822 4.0122) (end 35.47 3.7) (width 0.5) (layer "F.Cu") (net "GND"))
 (segment (start 9.1612 13.135) (end 8.525 13.135) (width 0.5) (layer "F.Cu") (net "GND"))
 (segment (start 27.525 30.635) (end 30.3497 30.635) (width 0.5) (layer "F.Cu") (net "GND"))
 (segment (start 30.3497 30.635) (end 31.6197 29.365) (width 0.5) (layer "F.Cu") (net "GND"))
 (segment (start 11.8991 10.3971) (end 9.1612 13.135) (width 0.5) (layer "F.Cu") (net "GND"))
 (segment (start 22.77 8.27) (end 22.77 3.7) (width 0.5) (layer "F.Cu") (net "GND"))
 (segment (start 31.6197 29.365) (end 32.475 29.365) (width 0.5) (layer "F.Cu") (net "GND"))
 (segment (start 35.7822 26.8641) (end 35.7822 4.0122) (width 0.5) (layer "F.Cu") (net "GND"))
 (segment (start 13.2771 10.3971) (end 11.8991 10.3971) (width 0.5) (layer "F.Cu") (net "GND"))
 (segment (start 13.475 10.595) (end 13.2771 10.3971) (width 0.5) (layer "F.Cu") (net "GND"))
 (segment (start 35 31.0837) (end 33.2813 29.365) (width 0.5) (layer "F.Cu") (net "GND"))
 (segment (start 36.8246 71.7554) (end 36.8246 39.3246) (width 0.5) (layer "F.Cu") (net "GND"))
 (segment (start 11.8991 5.5291) (end 11.8991 10.3971) (width 0.5) (layer "F.Cu") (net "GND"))
 (segment (start 32.475 29.365) (end 33.2813 29.365) (width 0.5) (layer "F.Cu") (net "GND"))
 (segment (start 25.5 11) (end 22.77 8.27) (width 0.5) (layer "F.Cu") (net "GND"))
 (segment (start 10.07 3.7) (end 11.8991 5.5291) (width 0.5) (layer "F.Cu") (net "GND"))
 (segment (start 36.8246 39.3246) (end 35 37.5) (width 0.5) (layer "F.Cu") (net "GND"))
 (segment (start 33.2813 29.365) (end 35.7822 26.8641) (width 0.5) (layer "F.Cu") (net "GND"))
 (segment (start 13.475 11.865) (end 13.475 10.595) (width 0.5) (layer "F.Cu") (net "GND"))
 (segment (start 35.5 73.08) (end 36.8246 71.7554) (width 0.5) (layer "F.Cu") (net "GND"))
 (segment (start 35 37.5) (end 32.4406 40.0594) (width 0.5) (layer "B.Cu") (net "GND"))
 (segment (start 35.47 3.7) (end 28.17 11) (width 0.5) (layer "B.Cu") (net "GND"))
 (segment (start 11.5653 2.2047) (end 10.07 3.7) (width 0.5) (layer "B.Cu") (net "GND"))
 (segment (start 28.17 11) (end 25.5 11) (width 0.5) (layer "B.Cu") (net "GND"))
 (segment (start 32.4406 40.0594) (end 24.6306 40.0594) (width 0.5) (layer "B.Cu") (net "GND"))
 (segment (start 21.2747 2.2047) (end 11.5653 2.2047) (width 0.5) (layer "B.Cu") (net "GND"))
 (segment (start 24.6306 40.0594) (end 20.35 44.34) (width 0.5) (layer "B.Cu") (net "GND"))
 (segment (start 22.77 3.7) (end 21.2747 2.2047) (width 0.5) (layer "B.Cu") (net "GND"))
 (segment (start 13.475 14.405) (end 18.3638 19.2938) (width 0.25) (layer "F.Cu") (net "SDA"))
 (segment (start 27.85 44.34) (end 27.85 36.53) (width 0.25) (layer "F.Cu") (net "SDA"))
 (segment (start 26.4816 45.7084) (end 27.85 44.34) (width 0.25) (layer "F.Cu") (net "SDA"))
 (segment (start 27.85 36.53) (end 32.475 31.905) (width 0.25) (layer "F.Cu") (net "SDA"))
 (segment (start 18.3638 44.2854) (end 19.7868 45.7084) (width 0.25) (layer "F.Cu") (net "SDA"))
 (segment (start 19.7868 45.7084) (end 26.4816 45.7084) (width 0.25) (layer "F.Cu") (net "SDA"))
 (segment (start 18.3638 19.2938) (end 18.3638 44.2854) (width 0.25) (layer "F.Cu") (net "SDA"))
 (segment (start 10.1751 14.405) (end 10.8101 13.77) (width 0.25) (layer "F.Cu") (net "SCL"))
 (segment (start 14.5669 13.77) (end 18.819 18.0221) (width 0.25) (layer "F.Cu") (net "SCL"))
 (segment (start 18.819 18.0221) (end 18.819 28.608) (width 0.25) (layer "F.Cu") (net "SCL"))
 (segment (start 18.819 28.608) (end 24.291 34.08) (width 0.25) (layer "F.Cu") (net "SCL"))
 (segment (start 10.8101 13.77) (end 14.5669 13.77) (width 0.25) (layer "F.Cu") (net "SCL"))
 (segment (start 27.525 31.905) (end 25.35 34.08) (width 0.25) (layer "F.Cu") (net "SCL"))
 (segment (start 24.291 34.08) (end 25.35 34.08) (width 0.25) (layer "F.Cu") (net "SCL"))
 (segment (start 25.35 34.08) (end 25.35 44.34) (width 0.25) (layer "F.Cu") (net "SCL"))
 (segment (start 8.525 14.405) (end 10.1751 14.405) (width 0.25) (layer "F.Cu") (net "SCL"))
 (segment (start 34.5 15.15) (end 34.5 26.871) (width 0.25) (layer "F.Cu") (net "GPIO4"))
 (via (at 34.5 26.871) (size 0.8) (drill 0.4) (layers "F.Cu" "B.Cu") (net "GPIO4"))
 (segment (start 36.2262 37.9814) (end 36.2262 28.5972) (width 0.25) (layer "B.Cu") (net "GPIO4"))
 (segment (start 22.85 44.34) (end 24.7523 42.4377) (width 0.25) (layer "B.Cu") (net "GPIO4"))
 (segment (start 36.2262 28.5972) (end 34.5 26.871) (width 0.25) (layer "B.Cu") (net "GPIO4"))
 (segment (start 31.7699 42.4377) (end 36.2262 37.9814) (width 0.25) (layer "B.Cu") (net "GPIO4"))
 (segment (start 24.7523 42.4377) (end 31.7699 42.4377) (width 0.25) (layer "B.Cu") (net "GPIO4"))
 (segment (start 22 18.1999) (end 20.2191 16.419) (width 0.25) (layer "F.Cu") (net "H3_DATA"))
 (segment (start 21.3455 9.8155) (end 23.7656 12.2356) (width 0.25) (layer "F.Cu") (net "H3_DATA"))
 (segment (start 25.9676 12.2356) (end 32.97 5.2332) (width 0.25) (layer "F.Cu") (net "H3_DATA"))
 (segment (start 22 29) (end 22 18.1999) (width 0.25) (layer "F.Cu") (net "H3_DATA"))
 (segment (start 32.97 5.2332) (end 32.97 3.7) (width 0.25) (layer "F.Cu") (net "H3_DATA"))
 (segment (start 19.9581 9.8155) (end 21.3455 9.8155) (width 0.25) (layer "F.Cu") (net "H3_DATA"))
 (segment (start 23.7656 12.2356) (end 25.9676 12.2356) (width 0.25) (layer "F.Cu") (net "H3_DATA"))
 (segment (start 19.2987 10.4749) (end 19.9581 9.8155) (width 0.25) (layer "F.Cu") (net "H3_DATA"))
 (segment (start 20.2191 12.6204) (end 19.2987 11.7) (width 0.25) (layer "F.Cu") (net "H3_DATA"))
 (segment (start 20.2191 16.419) (end 20.2191 12.6204) (width 0.25) (layer "F.Cu") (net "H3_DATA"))
 (segment (start 19.2987 11.7) (end 19.2987 10.4749) (width 0.25) (layer "F.Cu") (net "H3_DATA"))
 (segment (start 23.3 29) (end 27.16 29) (width 0.25) (layer "F.Cu") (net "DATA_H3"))
 (segment (start 27.16 29) (end 27.525 29.365) (width 0.25) (layer "F.Cu") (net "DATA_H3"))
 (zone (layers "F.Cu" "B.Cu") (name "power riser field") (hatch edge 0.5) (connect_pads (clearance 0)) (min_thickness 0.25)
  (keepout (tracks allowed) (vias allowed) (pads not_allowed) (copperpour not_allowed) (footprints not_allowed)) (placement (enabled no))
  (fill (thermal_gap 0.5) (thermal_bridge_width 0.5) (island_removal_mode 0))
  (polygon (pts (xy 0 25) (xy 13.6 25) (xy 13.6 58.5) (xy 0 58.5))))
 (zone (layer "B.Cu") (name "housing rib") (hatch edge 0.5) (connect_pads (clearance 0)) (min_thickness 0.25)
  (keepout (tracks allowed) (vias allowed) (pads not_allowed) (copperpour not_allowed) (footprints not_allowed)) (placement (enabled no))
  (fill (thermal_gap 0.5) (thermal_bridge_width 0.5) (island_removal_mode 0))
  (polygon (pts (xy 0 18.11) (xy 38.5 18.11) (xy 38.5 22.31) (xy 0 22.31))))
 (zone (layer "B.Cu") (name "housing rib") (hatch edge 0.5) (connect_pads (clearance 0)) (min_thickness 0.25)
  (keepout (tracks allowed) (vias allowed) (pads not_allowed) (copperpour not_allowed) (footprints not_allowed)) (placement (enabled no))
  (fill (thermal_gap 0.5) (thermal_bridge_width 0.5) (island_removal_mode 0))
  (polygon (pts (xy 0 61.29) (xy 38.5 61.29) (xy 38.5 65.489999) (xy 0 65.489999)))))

